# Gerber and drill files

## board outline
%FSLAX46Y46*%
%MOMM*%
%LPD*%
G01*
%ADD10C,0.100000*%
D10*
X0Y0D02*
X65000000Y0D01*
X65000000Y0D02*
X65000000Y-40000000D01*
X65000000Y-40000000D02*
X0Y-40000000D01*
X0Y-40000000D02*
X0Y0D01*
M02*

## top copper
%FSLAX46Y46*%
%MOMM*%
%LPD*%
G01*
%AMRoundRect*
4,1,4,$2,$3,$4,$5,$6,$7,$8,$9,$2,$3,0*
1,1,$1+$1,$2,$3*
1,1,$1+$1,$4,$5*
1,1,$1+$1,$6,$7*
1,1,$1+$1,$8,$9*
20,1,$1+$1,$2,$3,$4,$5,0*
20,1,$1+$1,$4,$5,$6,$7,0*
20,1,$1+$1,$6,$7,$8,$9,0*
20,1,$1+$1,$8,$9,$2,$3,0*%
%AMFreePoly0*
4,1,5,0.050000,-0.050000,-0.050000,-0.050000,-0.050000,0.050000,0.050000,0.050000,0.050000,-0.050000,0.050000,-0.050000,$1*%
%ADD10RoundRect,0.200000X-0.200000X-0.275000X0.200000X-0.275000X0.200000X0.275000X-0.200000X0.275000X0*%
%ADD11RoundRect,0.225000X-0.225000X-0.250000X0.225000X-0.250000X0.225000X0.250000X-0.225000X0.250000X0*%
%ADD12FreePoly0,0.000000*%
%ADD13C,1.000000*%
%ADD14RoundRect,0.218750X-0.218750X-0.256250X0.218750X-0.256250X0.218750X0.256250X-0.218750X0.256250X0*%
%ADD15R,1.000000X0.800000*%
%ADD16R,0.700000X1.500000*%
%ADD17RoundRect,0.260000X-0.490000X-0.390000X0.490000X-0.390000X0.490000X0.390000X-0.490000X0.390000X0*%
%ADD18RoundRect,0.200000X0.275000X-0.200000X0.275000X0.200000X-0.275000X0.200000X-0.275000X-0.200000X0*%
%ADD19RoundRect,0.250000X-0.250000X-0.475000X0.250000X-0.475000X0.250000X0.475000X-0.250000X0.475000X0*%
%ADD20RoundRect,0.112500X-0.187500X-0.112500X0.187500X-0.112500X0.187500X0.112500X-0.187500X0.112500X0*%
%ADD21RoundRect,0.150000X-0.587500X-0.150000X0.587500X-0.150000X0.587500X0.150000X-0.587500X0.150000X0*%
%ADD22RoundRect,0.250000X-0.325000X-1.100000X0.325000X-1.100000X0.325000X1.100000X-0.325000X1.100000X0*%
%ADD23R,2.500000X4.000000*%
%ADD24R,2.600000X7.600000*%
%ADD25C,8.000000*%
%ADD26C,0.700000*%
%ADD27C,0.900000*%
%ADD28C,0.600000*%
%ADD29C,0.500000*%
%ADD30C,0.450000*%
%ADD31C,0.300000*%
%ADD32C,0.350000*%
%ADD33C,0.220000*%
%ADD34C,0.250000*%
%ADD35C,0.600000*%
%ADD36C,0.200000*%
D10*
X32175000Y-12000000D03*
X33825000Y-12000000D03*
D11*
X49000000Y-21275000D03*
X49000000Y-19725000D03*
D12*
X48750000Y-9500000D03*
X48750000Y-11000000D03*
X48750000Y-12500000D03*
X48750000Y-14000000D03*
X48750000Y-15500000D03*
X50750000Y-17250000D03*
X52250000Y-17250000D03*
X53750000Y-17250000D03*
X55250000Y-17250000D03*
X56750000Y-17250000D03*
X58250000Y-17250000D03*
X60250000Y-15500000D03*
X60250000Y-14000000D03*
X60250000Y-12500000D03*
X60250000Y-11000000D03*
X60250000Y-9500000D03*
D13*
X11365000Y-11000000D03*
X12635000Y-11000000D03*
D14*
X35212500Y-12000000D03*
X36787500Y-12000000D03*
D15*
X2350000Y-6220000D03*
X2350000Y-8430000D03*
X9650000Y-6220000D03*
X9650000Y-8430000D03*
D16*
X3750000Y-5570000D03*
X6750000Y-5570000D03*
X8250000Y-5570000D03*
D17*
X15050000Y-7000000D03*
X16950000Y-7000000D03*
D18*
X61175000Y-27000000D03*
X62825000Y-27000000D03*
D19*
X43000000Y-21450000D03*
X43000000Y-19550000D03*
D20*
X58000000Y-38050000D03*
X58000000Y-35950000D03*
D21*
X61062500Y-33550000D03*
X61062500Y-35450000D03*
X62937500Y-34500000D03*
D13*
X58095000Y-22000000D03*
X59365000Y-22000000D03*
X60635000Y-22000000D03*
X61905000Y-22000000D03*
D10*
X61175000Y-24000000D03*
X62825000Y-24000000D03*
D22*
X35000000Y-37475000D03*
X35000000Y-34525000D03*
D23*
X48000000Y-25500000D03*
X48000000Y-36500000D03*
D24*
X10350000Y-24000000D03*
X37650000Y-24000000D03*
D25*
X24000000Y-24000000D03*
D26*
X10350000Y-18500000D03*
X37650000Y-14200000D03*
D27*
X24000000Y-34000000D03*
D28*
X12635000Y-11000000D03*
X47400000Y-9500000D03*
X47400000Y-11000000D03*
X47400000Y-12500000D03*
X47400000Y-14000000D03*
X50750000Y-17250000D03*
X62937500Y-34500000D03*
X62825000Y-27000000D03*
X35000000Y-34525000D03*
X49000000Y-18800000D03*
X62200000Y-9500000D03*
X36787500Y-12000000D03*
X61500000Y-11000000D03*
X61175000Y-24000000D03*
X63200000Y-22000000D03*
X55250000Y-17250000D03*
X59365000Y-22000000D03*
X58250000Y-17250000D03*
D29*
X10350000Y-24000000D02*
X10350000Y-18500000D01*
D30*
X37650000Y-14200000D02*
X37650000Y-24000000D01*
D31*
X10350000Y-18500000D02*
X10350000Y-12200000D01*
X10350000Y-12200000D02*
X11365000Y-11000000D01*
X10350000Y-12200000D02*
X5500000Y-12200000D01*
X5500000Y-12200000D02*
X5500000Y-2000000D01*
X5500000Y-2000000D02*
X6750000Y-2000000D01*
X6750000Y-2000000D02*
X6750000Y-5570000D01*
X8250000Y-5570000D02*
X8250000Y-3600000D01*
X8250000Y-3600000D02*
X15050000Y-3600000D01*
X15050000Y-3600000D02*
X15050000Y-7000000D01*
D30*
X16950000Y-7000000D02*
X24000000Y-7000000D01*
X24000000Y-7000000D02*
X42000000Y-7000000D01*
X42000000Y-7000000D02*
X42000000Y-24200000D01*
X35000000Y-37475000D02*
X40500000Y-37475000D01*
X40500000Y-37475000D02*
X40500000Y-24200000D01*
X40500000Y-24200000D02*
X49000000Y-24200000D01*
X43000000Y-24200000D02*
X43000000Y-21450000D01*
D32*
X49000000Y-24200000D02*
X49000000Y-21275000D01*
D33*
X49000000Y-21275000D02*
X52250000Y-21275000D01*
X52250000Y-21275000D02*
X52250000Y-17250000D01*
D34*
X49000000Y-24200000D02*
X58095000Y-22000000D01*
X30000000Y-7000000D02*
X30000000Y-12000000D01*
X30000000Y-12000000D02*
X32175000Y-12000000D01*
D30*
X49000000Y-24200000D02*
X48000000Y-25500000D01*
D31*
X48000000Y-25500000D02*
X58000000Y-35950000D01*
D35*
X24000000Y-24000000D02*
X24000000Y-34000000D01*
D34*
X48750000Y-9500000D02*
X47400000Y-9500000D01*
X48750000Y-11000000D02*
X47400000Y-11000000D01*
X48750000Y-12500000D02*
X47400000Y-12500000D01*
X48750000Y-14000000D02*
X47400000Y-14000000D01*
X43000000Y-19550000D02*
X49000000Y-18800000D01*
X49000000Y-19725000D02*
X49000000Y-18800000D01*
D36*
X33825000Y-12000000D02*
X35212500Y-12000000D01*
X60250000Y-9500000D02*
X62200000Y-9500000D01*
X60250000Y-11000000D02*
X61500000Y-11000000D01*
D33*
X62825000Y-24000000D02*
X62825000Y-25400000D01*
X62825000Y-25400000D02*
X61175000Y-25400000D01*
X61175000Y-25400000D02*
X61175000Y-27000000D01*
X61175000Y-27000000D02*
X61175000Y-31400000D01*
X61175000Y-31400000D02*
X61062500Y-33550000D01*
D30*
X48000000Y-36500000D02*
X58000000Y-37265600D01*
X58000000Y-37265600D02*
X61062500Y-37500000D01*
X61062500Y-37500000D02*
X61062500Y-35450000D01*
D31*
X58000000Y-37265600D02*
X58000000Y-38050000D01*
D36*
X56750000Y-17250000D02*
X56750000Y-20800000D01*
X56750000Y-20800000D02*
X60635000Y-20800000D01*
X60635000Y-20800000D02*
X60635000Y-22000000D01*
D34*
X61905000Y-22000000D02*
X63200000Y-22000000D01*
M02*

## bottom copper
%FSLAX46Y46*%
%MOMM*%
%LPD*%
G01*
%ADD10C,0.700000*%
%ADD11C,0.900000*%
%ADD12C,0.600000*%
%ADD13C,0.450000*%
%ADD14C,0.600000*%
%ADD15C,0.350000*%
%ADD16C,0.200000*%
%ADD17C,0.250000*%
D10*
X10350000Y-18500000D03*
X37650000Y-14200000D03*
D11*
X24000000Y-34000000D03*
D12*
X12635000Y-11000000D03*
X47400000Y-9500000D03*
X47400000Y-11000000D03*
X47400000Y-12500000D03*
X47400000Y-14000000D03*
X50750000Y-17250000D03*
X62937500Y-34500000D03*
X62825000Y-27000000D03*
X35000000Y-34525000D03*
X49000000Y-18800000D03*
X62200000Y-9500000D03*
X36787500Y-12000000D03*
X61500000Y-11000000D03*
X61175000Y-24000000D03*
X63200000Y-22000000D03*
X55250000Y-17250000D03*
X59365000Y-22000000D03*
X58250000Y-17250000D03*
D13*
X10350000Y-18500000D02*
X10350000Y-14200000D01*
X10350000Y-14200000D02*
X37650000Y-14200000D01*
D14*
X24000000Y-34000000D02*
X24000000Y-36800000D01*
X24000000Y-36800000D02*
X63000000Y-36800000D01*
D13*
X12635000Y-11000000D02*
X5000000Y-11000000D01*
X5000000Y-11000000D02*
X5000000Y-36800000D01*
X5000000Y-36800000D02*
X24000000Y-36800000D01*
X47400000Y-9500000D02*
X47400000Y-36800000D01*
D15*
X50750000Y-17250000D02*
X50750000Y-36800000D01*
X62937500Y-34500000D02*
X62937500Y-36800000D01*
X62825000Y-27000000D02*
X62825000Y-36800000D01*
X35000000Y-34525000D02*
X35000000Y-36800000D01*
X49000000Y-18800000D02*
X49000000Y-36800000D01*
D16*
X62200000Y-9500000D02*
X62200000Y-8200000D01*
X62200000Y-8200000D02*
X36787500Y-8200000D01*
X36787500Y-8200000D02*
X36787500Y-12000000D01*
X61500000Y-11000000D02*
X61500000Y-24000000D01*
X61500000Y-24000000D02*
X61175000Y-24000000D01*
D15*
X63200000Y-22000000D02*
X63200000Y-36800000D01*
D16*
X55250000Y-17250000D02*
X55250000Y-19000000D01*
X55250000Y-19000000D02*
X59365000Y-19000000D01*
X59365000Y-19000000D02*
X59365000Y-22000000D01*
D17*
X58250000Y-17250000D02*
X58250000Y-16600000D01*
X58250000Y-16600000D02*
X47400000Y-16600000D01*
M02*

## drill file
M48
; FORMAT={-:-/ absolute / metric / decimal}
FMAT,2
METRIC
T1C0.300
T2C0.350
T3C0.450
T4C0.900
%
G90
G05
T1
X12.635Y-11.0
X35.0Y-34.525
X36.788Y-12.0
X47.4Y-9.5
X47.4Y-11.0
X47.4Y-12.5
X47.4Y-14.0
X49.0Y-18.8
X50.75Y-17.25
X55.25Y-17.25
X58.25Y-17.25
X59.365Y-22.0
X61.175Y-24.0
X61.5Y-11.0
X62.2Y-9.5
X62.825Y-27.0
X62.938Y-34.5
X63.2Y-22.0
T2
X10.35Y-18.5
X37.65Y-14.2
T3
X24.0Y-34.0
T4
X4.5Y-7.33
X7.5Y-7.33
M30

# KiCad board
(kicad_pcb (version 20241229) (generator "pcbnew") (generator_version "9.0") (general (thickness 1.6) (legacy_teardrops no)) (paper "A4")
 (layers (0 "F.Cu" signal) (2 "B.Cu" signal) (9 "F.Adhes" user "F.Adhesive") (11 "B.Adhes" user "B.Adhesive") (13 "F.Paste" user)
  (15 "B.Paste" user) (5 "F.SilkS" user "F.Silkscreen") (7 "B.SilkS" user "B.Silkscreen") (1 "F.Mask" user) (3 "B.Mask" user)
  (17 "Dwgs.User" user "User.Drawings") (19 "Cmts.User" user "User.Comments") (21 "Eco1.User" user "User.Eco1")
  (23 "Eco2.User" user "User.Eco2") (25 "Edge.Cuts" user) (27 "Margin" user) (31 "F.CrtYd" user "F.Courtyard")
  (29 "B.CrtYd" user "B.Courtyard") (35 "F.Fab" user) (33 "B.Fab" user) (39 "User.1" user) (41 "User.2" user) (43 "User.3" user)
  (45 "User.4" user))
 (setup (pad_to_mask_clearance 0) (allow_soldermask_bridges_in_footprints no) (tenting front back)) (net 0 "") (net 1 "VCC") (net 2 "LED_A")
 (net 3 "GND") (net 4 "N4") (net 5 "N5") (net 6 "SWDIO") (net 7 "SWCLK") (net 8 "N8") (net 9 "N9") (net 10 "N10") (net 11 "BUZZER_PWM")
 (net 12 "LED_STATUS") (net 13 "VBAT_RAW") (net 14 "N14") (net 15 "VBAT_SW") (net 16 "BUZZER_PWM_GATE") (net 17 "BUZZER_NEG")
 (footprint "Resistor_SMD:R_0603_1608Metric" (layer "F.Cu") (at 33 12 0)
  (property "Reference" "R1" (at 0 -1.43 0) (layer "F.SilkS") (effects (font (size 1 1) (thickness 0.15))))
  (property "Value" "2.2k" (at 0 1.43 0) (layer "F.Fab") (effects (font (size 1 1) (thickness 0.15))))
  (pad "1" smd roundrect (at -0.825 0) (size 0.8 0.95) (layers "F.Cu" "F.Mask" "F.Paste") (roundrect_rratio 0.25) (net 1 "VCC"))
  (pad "2" smd roundrect (at 0.825 0) (size 0.8 0.95) (layers "F.Cu" "F.Mask" "F.Paste") (roundrect_rratio 0.25) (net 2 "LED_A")))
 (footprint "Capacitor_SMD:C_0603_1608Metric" (layer "F.Cu") (at 49 20.5 90)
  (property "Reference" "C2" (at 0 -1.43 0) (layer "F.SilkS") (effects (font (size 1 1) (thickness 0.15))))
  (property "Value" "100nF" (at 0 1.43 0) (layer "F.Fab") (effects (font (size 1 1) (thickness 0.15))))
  (pad "1" smd roundrect (at -0.775 0) (size 0.9 0.95) (layers "F.Cu" "F.Mask" "F.Paste") (roundrect_rratio 0.25) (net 1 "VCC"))
  (pad "2" smd roundrect (at 0.775 0) (size 0.9 0.95) (layers "F.Cu" "F.Mask" "F.Paste") (roundrect_rratio 0.25) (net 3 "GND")))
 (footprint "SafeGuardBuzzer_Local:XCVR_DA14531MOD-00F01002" (layer "F.Cu") (at 54.5 10.5 0)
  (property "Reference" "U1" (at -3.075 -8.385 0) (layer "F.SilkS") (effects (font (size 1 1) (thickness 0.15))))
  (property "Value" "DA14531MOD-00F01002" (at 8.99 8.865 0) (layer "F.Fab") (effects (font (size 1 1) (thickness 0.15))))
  (pad "J1" smd custom (at -5.75 -1) (size 0.1 0.1) (layers "F.Cu") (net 3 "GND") (options (clearance outline) (anchor rect)) (primitives))
  (pad "J2" smd custom (at -5.75 0.5) (size 0.1 0.1) (layers "F.Cu") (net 3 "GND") (options (clearance outline) (anchor rect)) (primitives))
  (pad "J3" smd custom (at -5.75 2) (size 0.1 0.1) (layers "F.Cu") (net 3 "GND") (options (clearance outline) (anchor rect)) (primitives))
  (pad "J4" smd custom (at -5.75 3.5) (size 0.1 0.1) (layers "F.Cu") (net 3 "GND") (options (clearance outline) (anchor rect)) (primitives))
  (pad "J5" smd custom (at -5.75 5) (size 0.1 0.1) (layers "F.Cu") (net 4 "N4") (options (clearance outline) (anchor rect)) (primitives))
  (pad "J6" smd custom (at -3.75 6.75) (size 0.1 0.1) (layers "F.Cu") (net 3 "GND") (options (clearance outline) (anchor rect)) (primitives))
  (pad "J7" smd custom (at -2.25 6.75) (size 0.1 0.1) (layers "F.Cu") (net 1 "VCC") (options (clearance outline) (anchor rect)) (primitives))
  (pad "J8" smd custom (at -0.75 6.75) (size 0.1 0.1) (layers "F.Cu") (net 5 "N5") (options (clearance outline) (anchor rect)) (primitives))
  (pad "J9" smd custom (at 0.75 6.75) (size 0.1 0.1) (layers "F.Cu") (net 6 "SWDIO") (options (clearance outline) (anchor rect))
   (primitives))
  (pad "J10" smd custom (at 2.25 6.75) (size 0.1 0.1) (layers "F.Cu") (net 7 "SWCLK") (options (clearance outline) (anchor rect))
   (primitives))
  (pad "J11" smd custom (at 3.75 6.75) (size 0.1 0.1) (layers "F.Cu") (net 3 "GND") (options (clearance outline) (anchor rect)) (primitives))
  (pad "J12" smd custom (at 5.75 5) (size 0.1 0.1) (layers "F.Cu") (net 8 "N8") (options (clearance outline) (anchor rect)) (primitives))
  (pad "J13" smd custom (at 5.75 3.5) (size 0.1 0.1) (layers "F.Cu") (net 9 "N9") (options (clearance outline) (anchor rect)) (primitives))
  (pad "J14" smd custom (at 5.75 2) (size 0.1 0.1) (layers "F.Cu") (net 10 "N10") (options (clearance outline) (anchor rect)) (primitives))
  (pad "J15" smd custom (at 5.75 0.5) (size 0.1 0.1) (layers "F.Cu") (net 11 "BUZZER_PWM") (options (clearance outline) (anchor rect))
   (primitives))
  (pad "J16" smd custom (at 5.75 -1) (size 0.1 0.1) (layers "F.Cu") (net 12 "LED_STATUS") (options (clearance outline) (anchor rect))
   (primitives))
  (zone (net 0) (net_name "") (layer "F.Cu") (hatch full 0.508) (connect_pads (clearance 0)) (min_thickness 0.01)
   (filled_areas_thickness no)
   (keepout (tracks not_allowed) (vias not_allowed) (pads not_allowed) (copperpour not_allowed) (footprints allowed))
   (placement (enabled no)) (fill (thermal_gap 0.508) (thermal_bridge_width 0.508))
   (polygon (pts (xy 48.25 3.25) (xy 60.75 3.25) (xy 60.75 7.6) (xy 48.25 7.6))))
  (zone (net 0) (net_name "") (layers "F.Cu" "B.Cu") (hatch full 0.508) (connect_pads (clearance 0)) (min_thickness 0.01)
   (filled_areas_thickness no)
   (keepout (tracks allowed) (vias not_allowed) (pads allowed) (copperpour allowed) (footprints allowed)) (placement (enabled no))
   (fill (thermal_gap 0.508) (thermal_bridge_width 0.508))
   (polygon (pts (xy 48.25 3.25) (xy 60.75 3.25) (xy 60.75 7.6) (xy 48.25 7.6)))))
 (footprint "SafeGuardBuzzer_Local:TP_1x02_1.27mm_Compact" (layer "F.Cu") (at 12 11 0)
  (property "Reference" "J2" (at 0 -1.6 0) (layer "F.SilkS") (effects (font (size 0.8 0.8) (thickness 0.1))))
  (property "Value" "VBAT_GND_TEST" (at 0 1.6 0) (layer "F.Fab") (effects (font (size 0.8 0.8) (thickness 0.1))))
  (pad "1" smd circle (at -0.635 0) (size 1 1) (layers "F.Cu" "F.Mask" "F.Paste") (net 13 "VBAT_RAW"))
  (pad "2" smd circle (at 0.635 0) (size 1 1) (layers "F.Cu" "F.Mask" "F.Paste") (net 3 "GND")))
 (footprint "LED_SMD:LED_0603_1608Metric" (layer "F.Cu") (at 36 12 0)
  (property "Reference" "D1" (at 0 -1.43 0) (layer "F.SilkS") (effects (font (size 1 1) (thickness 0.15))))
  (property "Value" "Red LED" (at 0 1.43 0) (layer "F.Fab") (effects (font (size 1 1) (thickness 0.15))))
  (pad "1" smd roundrect (at -0.7875 0) (size 0.875 0.95) (layers "F.Cu" "F.Mask" "F.Paste") (roundrect_rratio 0.25) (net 2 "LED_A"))
  (pad "2" smd roundrect (at 0.7875 0) (size 0.875 0.95) (layers "F.Cu" "F.Mask" "F.Paste") (roundrect_rratio 0.25) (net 12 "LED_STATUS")))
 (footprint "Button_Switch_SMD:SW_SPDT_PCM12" (layer "F.Cu") (at 6 7 0)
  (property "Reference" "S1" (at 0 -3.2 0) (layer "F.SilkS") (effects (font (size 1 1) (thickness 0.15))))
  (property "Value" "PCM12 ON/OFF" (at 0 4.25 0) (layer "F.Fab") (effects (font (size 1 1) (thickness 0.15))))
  (pad "" smd rect (at -3.65 -0.78) (size 1 0.8) (layers "F.Cu" "F.Mask" "F.Paste"))
  (pad "" smd rect (at -3.65 1.43) (size 1 0.8) (layers "F.Cu" "F.Mask" "F.Paste"))
  (pad "" np_thru_hole circle (at -1.5 0.33) (size 0.9 0.9) (drill 0.9) (layers "*.Cu" "*.Mask"))
  (pad "" np_thru_hole circle (at 1.5 0.33) (size 0.9 0.9) (drill 0.9) (layers "*.Cu" "*.Mask"))
  (pad "" smd rect (at 3.65 -0.78) (size 1 0.8) (layers "F.Cu" "F.Mask" "F.Paste"))
  (pad "" smd rect (at 3.65 1.43) (size 1 0.8) (layers "F.Cu" "F.Mask" "F.Paste"))
  (pad "1" smd rect (at -2.25 -1.43) (size 0.7 1.5) (layers "F.Cu" "F.Mask" "F.Paste") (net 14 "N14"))
  (pad "2" smd rect (at 0.75 -1.43) (size 0.7 1.5) (layers "F.Cu" "F.Mask" "F.Paste") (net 13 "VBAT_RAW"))
  (pad "3" smd rect (at 2.25 -1.43) (size 0.7 1.5) (layers "F.Cu" "F.Mask" "F.Paste") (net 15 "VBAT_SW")))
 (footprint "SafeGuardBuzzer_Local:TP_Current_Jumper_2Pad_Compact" (layer "F.Cu") (at 16 7 0)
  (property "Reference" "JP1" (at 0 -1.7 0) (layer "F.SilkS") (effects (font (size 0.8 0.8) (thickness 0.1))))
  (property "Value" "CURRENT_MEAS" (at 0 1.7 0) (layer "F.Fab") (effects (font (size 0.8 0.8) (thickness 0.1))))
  (pad "1" smd roundrect (at -0.95 0) (size 1.5 1.3) (layers "F.Cu" "F.Mask" "F.Paste") (roundrect_rratio 0.2) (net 15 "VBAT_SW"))
  (pad "2" smd roundrect (at 0.95 0) (size 1.5 1.3) (layers "F.Cu" "F.Mask" "F.Paste") (roundrect_rratio 0.2) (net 1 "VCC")))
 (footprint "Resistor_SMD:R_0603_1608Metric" (layer "F.Cu") (at 62 27 0)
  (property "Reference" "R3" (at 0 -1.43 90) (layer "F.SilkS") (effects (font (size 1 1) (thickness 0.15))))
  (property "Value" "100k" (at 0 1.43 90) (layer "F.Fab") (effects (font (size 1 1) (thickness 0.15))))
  (pad "1" smd roundrect (at -0.825 0 90) (size 0.8 0.95) (layers "F.Cu" "F.Mask" "F.Paste") (roundrect_rratio 0.25)
   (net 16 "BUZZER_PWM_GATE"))
  (pad "2" smd roundrect (at 0.825 0 90) (size 0.8 0.95) (layers "F.Cu" "F.Mask" "F.Paste") (roundrect_rratio 0.25) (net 3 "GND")))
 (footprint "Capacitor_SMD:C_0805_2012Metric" (layer "F.Cu") (at 43 20.5 90)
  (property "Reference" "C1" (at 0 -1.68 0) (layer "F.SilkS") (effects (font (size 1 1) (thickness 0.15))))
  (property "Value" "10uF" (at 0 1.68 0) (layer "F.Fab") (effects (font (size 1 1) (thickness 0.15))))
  (pad "1" smd roundrect (at -0.95 0) (size 1 1.45) (layers "F.Cu" "F.Mask" "F.Paste") (roundrect_rratio 0.25) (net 1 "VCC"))
  (pad "2" smd roundrect (at 0.95 0) (size 1 1.45) (layers "F.Cu" "F.Mask" "F.Paste") (roundrect_rratio 0.25) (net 3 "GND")))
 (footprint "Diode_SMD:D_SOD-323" (layer "F.Cu") (at 58 37 90)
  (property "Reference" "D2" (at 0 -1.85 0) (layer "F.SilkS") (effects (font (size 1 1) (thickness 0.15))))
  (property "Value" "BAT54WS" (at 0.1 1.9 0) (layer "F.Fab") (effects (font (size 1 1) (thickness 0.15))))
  (pad "1" smd roundrect (at -1.05 0) (size 0.6 0.45) (layers "F.Cu" "F.Mask" "F.Paste") (roundrect_rratio 0.25) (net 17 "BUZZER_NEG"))
  (pad "2" smd roundrect (at 1.05 0) (size 0.6 0.45) (layers "F.Cu" "F.Mask" "F.Paste") (roundrect_rratio 0.25) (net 1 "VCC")))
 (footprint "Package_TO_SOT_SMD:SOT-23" (layer "F.Cu") (at 62 34.5 0)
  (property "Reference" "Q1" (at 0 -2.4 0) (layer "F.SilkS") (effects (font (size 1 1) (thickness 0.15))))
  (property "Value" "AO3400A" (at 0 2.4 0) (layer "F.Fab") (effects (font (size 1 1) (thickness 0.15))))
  (pad "1" smd roundrect (at -0.9375 -0.95) (size 1.475 0.6) (layers "F.Cu" "F.Mask" "F.Paste") (roundrect_rratio 0.25)
   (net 16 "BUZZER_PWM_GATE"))
  (pad "2" smd roundrect (at -0.9375 0.95) (size 1.475 0.6) (layers "F.Cu" "F.Mask" "F.Paste") (roundrect_rratio 0.25) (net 17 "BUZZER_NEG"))
  (pad "3" smd roundrect (at 0.9375 0) (size 1.475 0.6) (layers "F.Cu" "F.Mask" "F.Paste") (roundrect_rratio 0.25) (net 3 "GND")))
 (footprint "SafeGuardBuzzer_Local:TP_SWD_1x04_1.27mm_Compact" (layer "F.Cu") (at 60 22 0)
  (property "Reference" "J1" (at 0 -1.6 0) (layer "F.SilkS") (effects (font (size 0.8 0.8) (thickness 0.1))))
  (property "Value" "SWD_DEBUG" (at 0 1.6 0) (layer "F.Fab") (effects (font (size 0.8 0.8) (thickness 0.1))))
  (pad "1" smd circle (at -1.905 0) (size 1 1) (layers "F.Cu" "F.Mask" "F.Paste") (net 1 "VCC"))
  (pad "2" smd circle (at -0.635 0) (size 1 1) (layers "F.Cu" "F.Mask" "F.Paste") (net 6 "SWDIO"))
  (pad "3" smd circle (at 0.635 0) (size 1 1) (layers "F.Cu" "F.Mask" "F.Paste") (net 7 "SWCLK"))
  (pad "4" smd circle (at 1.905 0) (size 1 1) (layers "F.Cu" "F.Mask" "F.Paste") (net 3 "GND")))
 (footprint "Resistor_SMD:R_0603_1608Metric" (layer "F.Cu") (at 62 24 0)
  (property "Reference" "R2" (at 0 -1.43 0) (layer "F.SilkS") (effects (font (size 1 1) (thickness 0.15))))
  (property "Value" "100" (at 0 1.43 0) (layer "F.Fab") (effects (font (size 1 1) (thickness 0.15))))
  (pad "1" smd roundrect (at -0.825 0) (size 0.8 0.95) (layers "F.Cu" "F.Mask" "F.Paste") (roundrect_rratio 0.25) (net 11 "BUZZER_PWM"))
  (pad "2" smd roundrect (at 0.825 0) (size 0.8 0.95) (layers "F.Cu" "F.Mask" "F.Paste") (roundrect_rratio 0.25) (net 16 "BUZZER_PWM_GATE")))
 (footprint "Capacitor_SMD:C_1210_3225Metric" (layer "F.Cu") (at 35 36 90)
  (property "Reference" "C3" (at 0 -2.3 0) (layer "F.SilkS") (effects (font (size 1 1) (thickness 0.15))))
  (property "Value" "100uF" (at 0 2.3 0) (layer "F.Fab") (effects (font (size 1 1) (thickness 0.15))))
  (pad "1" smd roundrect (at -1.475 0) (size 1.15 2.7) (layers "F.Cu" "F.Mask" "F.Paste") (roundrect_rratio 0.217391) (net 1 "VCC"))
  (pad "2" smd roundrect (at 1.475 0) (size 1.15 2.7) (layers "F.Cu" "F.Mask" "F.Paste") (roundrect_rratio 0.217391) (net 3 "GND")))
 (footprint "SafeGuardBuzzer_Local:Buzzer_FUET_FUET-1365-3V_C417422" (layer "F.Cu") (at 48 31 0)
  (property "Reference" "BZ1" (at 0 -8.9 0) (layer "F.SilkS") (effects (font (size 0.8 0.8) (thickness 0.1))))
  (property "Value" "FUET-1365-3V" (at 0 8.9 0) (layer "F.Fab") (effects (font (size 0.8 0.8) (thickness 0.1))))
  (pad "1" smd rect (at 0 -5.5) (size 2.5 4) (layers "F.Cu" "F.Mask" "F.Paste") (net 1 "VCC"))
  (pad "2" smd rect (at 0 5.5) (size 2.5 4) (layers "F.Cu" "F.Mask" "F.Paste") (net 17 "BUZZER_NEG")))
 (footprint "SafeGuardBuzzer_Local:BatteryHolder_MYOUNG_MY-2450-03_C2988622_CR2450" (layer "F.Cu") (at 24 24 0)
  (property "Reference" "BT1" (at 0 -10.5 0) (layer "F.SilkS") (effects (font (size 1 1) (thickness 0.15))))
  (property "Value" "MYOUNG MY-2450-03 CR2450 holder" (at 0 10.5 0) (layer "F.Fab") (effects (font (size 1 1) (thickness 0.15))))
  (pad "1" smd rect (at -13.65 0) (size 2.6 7.6) (layers "F.Cu" "F.Mask" "F.Paste") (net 13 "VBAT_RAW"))
  (pad "1" smd rect (at 13.65 0) (size 2.6 7.6) (layers "F.Cu" "F.Mask" "F.Paste") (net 13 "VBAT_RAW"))
  (pad "2" smd circle (at 0 0) (size 8 8) (layers "F.Cu" "F.Mask") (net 3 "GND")))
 (gr_line (start 0 0) (end 65 0) (stroke (width 0.1) (type default)) (layer "Edge.Cuts"))
 (gr_line (start 65 0) (end 65 40) (stroke (width 0.1) (type default)) (layer "Edge.Cuts"))
 (gr_line (start 65 40) (end 0 40) (stroke (width 0.1) (type default)) (layer "Edge.Cuts"))
 (gr_line (start 0 40) (end 0 0) (stroke (width 0.1) (type default)) (layer "Edge.Cuts"))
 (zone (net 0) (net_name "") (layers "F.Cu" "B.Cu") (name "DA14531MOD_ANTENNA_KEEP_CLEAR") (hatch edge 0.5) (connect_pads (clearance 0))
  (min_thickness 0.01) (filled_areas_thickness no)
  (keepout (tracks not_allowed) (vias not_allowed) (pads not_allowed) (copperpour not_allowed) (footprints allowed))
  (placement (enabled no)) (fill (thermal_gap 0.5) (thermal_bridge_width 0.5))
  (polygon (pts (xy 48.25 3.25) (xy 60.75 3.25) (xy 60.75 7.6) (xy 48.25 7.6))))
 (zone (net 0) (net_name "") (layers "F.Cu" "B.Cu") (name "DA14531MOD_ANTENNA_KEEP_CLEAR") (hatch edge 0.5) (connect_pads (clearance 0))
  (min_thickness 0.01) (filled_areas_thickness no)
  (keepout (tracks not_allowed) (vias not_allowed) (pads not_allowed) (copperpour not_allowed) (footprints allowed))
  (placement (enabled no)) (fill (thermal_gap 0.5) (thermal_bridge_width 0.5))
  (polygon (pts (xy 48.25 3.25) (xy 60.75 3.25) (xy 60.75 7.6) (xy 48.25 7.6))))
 (via (at 10.3500 18.5000) (size 0.7000) (drill 0.3500) (layers "F.Cu" "B.Cu") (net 13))
 (segment (start 10.3500 24.0000) (end 10.3500 18.5000) (width 0.5000) (layer "F.Cu") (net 13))
 (segment (start 10.3500 18.5000) (end 10.3500 14.2000) (width 0.4500) (layer "B.Cu") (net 13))
 (segment (start 10.3500 14.2000) (end 37.6500 14.2000) (width 0.4500) (layer "B.Cu") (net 13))
 (via (at 37.6500 14.2000) (size 0.7000) (drill 0.3500) (layers "F.Cu" "B.Cu") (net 13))
 (segment (start 37.6500 14.2000) (end 37.6500 24.0000) (width 0.4500) (layer "F.Cu") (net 13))
 (segment (start 10.3500 18.5000) (end 10.3500 12.2000) (width 0.3000) (layer "F.Cu") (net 13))
 (segment (start 10.3500 12.2000) (end 11.3650 11.0000) (width 0.3000) (layer "F.Cu") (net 13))
 (segment (start 10.3500 12.2000) (end 5.5000 12.2000) (width 0.3000) (layer "F.Cu") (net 13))
 (segment (start 5.5000 12.2000) (end 5.5000 2.0000) (width 0.3000) (layer "F.Cu") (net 13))
 (segment (start 5.5000 2.0000) (end 6.7500 2.0000) (width 0.3000) (layer "F.Cu") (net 13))
 (segment (start 6.7500 2.0000) (end 6.7500 5.5700) (width 0.3000) (layer "F.Cu") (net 13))
 (segment (start 8.2500 5.5700) (end 8.2500 3.6000) (width 0.3000) (layer "F.Cu") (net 15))
 (segment (start 8.2500 3.6000) (end 15.0500 3.6000) (width 0.3000) (layer "F.Cu") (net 15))
 (segment (start 15.0500 3.6000) (end 15.0500 7.0000) (width 0.3000) (layer "F.Cu") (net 15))
 (segment (start 16.9500 7.0000) (end 24.0000 7.0000) (width 0.4500) (layer "F.Cu") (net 1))
 (segment (start 24.0000 7.0000) (end 42.0000 7.0000) (width 0.4500) (layer "F.Cu") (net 1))
 (segment (start 42.0000 7.0000) (end 42.0000 24.2000) (width 0.4500) (layer "F.Cu") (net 1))
 (segment (start 35.0000 37.4750) (end 40.5000 37.4750) (width 0.4500) (layer "F.Cu") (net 1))
 (segment (start 40.5000 37.4750) (end 40.5000 24.2000) (width 0.4500) (layer "F.Cu") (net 1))
 (segment (start 40.5000 24.2000) (end 49.0000 24.2000) (width 0.4500) (layer "F.Cu") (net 1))
 (segment (start 43.0000 24.2000) (end 43.0000 21.4500) (width 0.4500) (layer "F.Cu") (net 1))
 (segment (start 49.0000 24.2000) (end 49.0000 21.2750) (width 0.3500) (layer "F.Cu") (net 1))
 (segment (start 49.0000 21.2750) (end 52.2500 21.2750) (width 0.2200) (layer "F.Cu") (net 1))
 (segment (start 52.2500 21.2750) (end 52.2500 17.2500) (width 0.2200) (layer "F.Cu") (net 1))
 (segment (start 49.0000 24.2000) (end 58.0950 22.0000) (width 0.2500) (layer "F.Cu") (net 1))
 (segment (start 30.0000 7.0000) (end 30.0000 12.0000) (width 0.2500) (layer "F.Cu") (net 1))
 (segment (start 30.0000 12.0000) (end 32.1750 12.0000) (width 0.2500) (layer "F.Cu") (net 1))
 (segment (start 49.0000 24.2000) (end 48.0000 25.5000) (width 0.4500) (layer "F.Cu") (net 1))
 (segment (start 48.0000 25.5000) (end 58.0000 35.9500) (width 0.3000) (layer "F.Cu") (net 1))
 (segment (start 24.0000 24.0000) (end 24.0000 34.0000) (width 0.6000) (layer "F.Cu") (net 3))
 (via (at 24.0000 34.0000) (size 0.9000) (drill 0.4500) (layers "F.Cu" "B.Cu") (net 3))
 (segment (start 24.0000 34.0000) (end 24.0000 36.8000) (width 0.6000) (layer "B.Cu") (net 3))
 (segment (start 24.0000 36.8000) (end 63.0000 36.8000) (width 0.6000) (layer "B.Cu") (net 3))
 (via (at 12.6350 11.0000) (size 0.6000) (drill 0.3000) (layers "F.Cu" "B.Cu") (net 3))
 (segment (start 12.6350 11.0000) (end 5.0000 11.0000) (width 0.4500) (layer "B.Cu") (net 3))
 (segment (start 5.0000 11.0000) (end 5.0000 36.8000) (width 0.4500) (layer "B.Cu") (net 3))
 (segment (start 5.0000 36.8000) (end 24.0000 36.8000) (width 0.4500) (layer "B.Cu") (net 3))
 (segment (start 47.4000 9.5000) (end 47.4000 36.8000) (width 0.4500) (layer "B.Cu") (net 3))
 (via (at 47.4000 9.5000) (size 0.6000) (drill 0.3000) (layers "F.Cu" "B.Cu") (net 3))
 (segment (start 48.7500 9.5000) (end 47.4000 9.5000) (width 0.2500) (layer "F.Cu") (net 3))
 (via (at 47.4000 11.0000) (size 0.6000) (drill 0.3000) (layers "F.Cu" "B.Cu") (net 3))
 (segment (start 48.7500 11.0000) (end 47.4000 11.0000) (width 0.2500) (layer "F.Cu") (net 3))
 (via (at 47.4000 12.5000) (size 0.6000) (drill 0.3000) (layers "F.Cu" "B.Cu") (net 3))
 (segment (start 48.7500 12.5000) (end 47.4000 12.5000) (width 0.2500) (layer "F.Cu") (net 3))
 (via (at 47.4000 14.0000) (size 0.6000) (drill 0.3000) (layers "F.Cu" "B.Cu") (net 3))
 (segment (start 48.7500 14.0000) (end 47.4000 14.0000) (width 0.2500) (layer "F.Cu") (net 3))
 (via (at 50.7500 17.2500) (size 0.6000) (drill 0.3000) (layers "F.Cu" "B.Cu") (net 3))
 (segment (start 50.7500 17.2500) (end 50.7500 36.8000) (width 0.3500) (layer "B.Cu") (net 3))
 (via (at 62.9375 34.5000) (size 0.6000) (drill 0.3000) (layers "F.Cu" "B.Cu") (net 3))
 (segment (start 62.9375 34.5000) (end 62.9375 36.8000) (width 0.3500) (layer "B.Cu") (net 3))
 (via (at 62.8250 27.0000) (size 0.6000) (drill 0.3000) (layers "F.Cu" "B.Cu") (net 3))
 (segment (start 62.8250 27.0000) (end 62.8250 36.8000) (width 0.3500) (layer "B.Cu") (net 3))
 (via (at 35.0000 34.5250) (size 0.6000) (drill 0.3000) (layers "F.Cu" "B.Cu") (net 3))
 (segment (start 35.0000 34.5250) (end 35.0000 36.8000) (width 0.3500) (layer "B.Cu") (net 3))
 (via (at 49.0000 18.8000) (size 0.6000) (drill 0.3000) (layers "F.Cu" "B.Cu") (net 3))
 (segment (start 49.0000 18.8000) (end 49.0000 36.8000) (width 0.3500) (layer "B.Cu") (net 3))
 (segment (start 43.0000 19.5500) (end 49.0000 18.8000) (width 0.2500) (layer "F.Cu") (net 3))
 (segment (start 49.0000 19.7250) (end 49.0000 18.8000) (width 0.2500) (layer "F.Cu") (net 3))
 (segment (start 33.8250 12.0000) (end 35.2125 12.0000) (width 0.2000) (layer "F.Cu") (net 2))
 (via (at 62.2000 9.5000) (size 0.6000) (drill 0.3000) (layers "F.Cu" "B.Cu") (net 12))
 (via (at 36.7875 12.0000) (size 0.6000) (drill 0.3000) (layers "F.Cu" "B.Cu") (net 12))
 (segment (start 60.2500 9.5000) (end 62.2000 9.5000) (width 0.2000) (layer "F.Cu") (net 12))
 (segment (start 62.2000 9.5000) (end 62.2000 8.2000) (width 0.2000) (layer "B.Cu") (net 12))
 (segment (start 62.2000 8.2000) (end 36.7875 8.2000) (width 0.2000) (layer "B.Cu") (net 12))
 (segment (start 36.7875 8.2000) (end 36.7875 12.0000) (width 0.2000) (layer "B.Cu") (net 12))
 (via (at 61.5000 11.0000) (size 0.6000) (drill 0.3000) (layers "F.Cu" "B.Cu") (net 11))
 (via (at 61.1750 24.0000) (size 0.6000) (drill 0.3000) (layers "F.Cu" "B.Cu") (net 11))
 (segment (start 60.2500 11.0000) (end 61.5000 11.0000) (width 0.2000) (layer "F.Cu") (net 11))
 (segment (start 61.5000 11.0000) (end 61.5000 24.0000) (width 0.2000) (layer "B.Cu") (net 11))
 (segment (start 61.5000 24.0000) (end 61.1750 24.0000) (width 0.2000) (layer "B.Cu") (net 11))
 (segment (start 62.8250 24.0000) (end 62.8250 25.4000) (width 0.2200) (layer "F.Cu") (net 16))
 (segment (start 62.8250 25.4000) (end 61.1750 25.4000) (width 0.2200) (layer "F.Cu") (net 16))
 (segment (start 61.1750 25.4000) (end 61.1750 27.0000) (width 0.2200) (layer "F.Cu") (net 16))
 (segment (start 61.1750 27.0000) (end 61.1750 31.4000) (width 0.2200) (layer "F.Cu") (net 16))
 (segment (start 61.1750 31.4000) (end 61.0625 33.5500) (width 0.2200) (layer "F.Cu") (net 16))
 (segment (start 48.0000 36.5000) (end 58.0000 37.2656) (width 0.4500) (layer "F.Cu") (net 17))
 (segment (start 58.0000 37.2656) (end 61.0625 37.5000) (width 0.4500) (layer "F.Cu") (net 17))
 (segment (start 61.0625 37.5000) (end 61.0625 35.4500) (width 0.4500) (layer "F.Cu") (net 17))
 (segment (start 58.0000 37.2656) (end 58.0000 38.0500) (width 0.3000) (layer "F.Cu") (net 17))
 (segment (start 56.7500 17.2500) (end 56.7500 20.8000) (width 0.2000) (layer "F.Cu") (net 7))
 (segment (start 56.7500 20.8000) (end 60.6350 20.8000) (width 0.2000) (layer "F.Cu") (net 7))
 (segment (start 60.6350 20.8000) (end 60.6350 22.0000) (width 0.2000) (layer "F.Cu") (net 7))
 (segment (start 61.9050 22.0000) (end 63.2000 22.0000) (width 0.2500) (layer "F.Cu") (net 3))
 (via (at 63.2000 22.0000) (size 0.6000) (drill 0.3000) (layers "F.Cu" "B.Cu") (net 3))
 (segment (start 63.2000 22.0000) (end 63.2000 36.8000) (width 0.3500) (layer "B.Cu") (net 3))
 (via (at 55.2500 17.2500) (size 0.6000) (drill 0.3000) (layers "F.Cu" "B.Cu") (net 6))
 (via (at 59.3650 22.0000) (size 0.6000) (drill 0.3000) (layers "F.Cu" "B.Cu") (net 6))
 (segment (start 55.2500 17.2500) (end 55.2500 19.0000) (width 0.2000) (layer "B.Cu") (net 6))
 (segment (start 55.2500 19.0000) (end 59.3650 19.0000) (width 0.2000) (layer "B.Cu") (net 6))
 (segment (start 59.3650 19.0000) (end 59.3650 22.0000) (width 0.2000) (layer "B.Cu") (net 6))
 (via (at 58.2500 17.2500) (size 0.6000) (drill 0.3000) (layers "F.Cu" "B.Cu") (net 3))
 (segment (start 58.2500 17.2500) (end 58.2500 16.6000) (width 0.2500) (layer "B.Cu") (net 3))
 (segment (start 58.2500 16.6000) (end 47.4000 16.6000) (width 0.2500) (layer "B.Cu") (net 3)))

